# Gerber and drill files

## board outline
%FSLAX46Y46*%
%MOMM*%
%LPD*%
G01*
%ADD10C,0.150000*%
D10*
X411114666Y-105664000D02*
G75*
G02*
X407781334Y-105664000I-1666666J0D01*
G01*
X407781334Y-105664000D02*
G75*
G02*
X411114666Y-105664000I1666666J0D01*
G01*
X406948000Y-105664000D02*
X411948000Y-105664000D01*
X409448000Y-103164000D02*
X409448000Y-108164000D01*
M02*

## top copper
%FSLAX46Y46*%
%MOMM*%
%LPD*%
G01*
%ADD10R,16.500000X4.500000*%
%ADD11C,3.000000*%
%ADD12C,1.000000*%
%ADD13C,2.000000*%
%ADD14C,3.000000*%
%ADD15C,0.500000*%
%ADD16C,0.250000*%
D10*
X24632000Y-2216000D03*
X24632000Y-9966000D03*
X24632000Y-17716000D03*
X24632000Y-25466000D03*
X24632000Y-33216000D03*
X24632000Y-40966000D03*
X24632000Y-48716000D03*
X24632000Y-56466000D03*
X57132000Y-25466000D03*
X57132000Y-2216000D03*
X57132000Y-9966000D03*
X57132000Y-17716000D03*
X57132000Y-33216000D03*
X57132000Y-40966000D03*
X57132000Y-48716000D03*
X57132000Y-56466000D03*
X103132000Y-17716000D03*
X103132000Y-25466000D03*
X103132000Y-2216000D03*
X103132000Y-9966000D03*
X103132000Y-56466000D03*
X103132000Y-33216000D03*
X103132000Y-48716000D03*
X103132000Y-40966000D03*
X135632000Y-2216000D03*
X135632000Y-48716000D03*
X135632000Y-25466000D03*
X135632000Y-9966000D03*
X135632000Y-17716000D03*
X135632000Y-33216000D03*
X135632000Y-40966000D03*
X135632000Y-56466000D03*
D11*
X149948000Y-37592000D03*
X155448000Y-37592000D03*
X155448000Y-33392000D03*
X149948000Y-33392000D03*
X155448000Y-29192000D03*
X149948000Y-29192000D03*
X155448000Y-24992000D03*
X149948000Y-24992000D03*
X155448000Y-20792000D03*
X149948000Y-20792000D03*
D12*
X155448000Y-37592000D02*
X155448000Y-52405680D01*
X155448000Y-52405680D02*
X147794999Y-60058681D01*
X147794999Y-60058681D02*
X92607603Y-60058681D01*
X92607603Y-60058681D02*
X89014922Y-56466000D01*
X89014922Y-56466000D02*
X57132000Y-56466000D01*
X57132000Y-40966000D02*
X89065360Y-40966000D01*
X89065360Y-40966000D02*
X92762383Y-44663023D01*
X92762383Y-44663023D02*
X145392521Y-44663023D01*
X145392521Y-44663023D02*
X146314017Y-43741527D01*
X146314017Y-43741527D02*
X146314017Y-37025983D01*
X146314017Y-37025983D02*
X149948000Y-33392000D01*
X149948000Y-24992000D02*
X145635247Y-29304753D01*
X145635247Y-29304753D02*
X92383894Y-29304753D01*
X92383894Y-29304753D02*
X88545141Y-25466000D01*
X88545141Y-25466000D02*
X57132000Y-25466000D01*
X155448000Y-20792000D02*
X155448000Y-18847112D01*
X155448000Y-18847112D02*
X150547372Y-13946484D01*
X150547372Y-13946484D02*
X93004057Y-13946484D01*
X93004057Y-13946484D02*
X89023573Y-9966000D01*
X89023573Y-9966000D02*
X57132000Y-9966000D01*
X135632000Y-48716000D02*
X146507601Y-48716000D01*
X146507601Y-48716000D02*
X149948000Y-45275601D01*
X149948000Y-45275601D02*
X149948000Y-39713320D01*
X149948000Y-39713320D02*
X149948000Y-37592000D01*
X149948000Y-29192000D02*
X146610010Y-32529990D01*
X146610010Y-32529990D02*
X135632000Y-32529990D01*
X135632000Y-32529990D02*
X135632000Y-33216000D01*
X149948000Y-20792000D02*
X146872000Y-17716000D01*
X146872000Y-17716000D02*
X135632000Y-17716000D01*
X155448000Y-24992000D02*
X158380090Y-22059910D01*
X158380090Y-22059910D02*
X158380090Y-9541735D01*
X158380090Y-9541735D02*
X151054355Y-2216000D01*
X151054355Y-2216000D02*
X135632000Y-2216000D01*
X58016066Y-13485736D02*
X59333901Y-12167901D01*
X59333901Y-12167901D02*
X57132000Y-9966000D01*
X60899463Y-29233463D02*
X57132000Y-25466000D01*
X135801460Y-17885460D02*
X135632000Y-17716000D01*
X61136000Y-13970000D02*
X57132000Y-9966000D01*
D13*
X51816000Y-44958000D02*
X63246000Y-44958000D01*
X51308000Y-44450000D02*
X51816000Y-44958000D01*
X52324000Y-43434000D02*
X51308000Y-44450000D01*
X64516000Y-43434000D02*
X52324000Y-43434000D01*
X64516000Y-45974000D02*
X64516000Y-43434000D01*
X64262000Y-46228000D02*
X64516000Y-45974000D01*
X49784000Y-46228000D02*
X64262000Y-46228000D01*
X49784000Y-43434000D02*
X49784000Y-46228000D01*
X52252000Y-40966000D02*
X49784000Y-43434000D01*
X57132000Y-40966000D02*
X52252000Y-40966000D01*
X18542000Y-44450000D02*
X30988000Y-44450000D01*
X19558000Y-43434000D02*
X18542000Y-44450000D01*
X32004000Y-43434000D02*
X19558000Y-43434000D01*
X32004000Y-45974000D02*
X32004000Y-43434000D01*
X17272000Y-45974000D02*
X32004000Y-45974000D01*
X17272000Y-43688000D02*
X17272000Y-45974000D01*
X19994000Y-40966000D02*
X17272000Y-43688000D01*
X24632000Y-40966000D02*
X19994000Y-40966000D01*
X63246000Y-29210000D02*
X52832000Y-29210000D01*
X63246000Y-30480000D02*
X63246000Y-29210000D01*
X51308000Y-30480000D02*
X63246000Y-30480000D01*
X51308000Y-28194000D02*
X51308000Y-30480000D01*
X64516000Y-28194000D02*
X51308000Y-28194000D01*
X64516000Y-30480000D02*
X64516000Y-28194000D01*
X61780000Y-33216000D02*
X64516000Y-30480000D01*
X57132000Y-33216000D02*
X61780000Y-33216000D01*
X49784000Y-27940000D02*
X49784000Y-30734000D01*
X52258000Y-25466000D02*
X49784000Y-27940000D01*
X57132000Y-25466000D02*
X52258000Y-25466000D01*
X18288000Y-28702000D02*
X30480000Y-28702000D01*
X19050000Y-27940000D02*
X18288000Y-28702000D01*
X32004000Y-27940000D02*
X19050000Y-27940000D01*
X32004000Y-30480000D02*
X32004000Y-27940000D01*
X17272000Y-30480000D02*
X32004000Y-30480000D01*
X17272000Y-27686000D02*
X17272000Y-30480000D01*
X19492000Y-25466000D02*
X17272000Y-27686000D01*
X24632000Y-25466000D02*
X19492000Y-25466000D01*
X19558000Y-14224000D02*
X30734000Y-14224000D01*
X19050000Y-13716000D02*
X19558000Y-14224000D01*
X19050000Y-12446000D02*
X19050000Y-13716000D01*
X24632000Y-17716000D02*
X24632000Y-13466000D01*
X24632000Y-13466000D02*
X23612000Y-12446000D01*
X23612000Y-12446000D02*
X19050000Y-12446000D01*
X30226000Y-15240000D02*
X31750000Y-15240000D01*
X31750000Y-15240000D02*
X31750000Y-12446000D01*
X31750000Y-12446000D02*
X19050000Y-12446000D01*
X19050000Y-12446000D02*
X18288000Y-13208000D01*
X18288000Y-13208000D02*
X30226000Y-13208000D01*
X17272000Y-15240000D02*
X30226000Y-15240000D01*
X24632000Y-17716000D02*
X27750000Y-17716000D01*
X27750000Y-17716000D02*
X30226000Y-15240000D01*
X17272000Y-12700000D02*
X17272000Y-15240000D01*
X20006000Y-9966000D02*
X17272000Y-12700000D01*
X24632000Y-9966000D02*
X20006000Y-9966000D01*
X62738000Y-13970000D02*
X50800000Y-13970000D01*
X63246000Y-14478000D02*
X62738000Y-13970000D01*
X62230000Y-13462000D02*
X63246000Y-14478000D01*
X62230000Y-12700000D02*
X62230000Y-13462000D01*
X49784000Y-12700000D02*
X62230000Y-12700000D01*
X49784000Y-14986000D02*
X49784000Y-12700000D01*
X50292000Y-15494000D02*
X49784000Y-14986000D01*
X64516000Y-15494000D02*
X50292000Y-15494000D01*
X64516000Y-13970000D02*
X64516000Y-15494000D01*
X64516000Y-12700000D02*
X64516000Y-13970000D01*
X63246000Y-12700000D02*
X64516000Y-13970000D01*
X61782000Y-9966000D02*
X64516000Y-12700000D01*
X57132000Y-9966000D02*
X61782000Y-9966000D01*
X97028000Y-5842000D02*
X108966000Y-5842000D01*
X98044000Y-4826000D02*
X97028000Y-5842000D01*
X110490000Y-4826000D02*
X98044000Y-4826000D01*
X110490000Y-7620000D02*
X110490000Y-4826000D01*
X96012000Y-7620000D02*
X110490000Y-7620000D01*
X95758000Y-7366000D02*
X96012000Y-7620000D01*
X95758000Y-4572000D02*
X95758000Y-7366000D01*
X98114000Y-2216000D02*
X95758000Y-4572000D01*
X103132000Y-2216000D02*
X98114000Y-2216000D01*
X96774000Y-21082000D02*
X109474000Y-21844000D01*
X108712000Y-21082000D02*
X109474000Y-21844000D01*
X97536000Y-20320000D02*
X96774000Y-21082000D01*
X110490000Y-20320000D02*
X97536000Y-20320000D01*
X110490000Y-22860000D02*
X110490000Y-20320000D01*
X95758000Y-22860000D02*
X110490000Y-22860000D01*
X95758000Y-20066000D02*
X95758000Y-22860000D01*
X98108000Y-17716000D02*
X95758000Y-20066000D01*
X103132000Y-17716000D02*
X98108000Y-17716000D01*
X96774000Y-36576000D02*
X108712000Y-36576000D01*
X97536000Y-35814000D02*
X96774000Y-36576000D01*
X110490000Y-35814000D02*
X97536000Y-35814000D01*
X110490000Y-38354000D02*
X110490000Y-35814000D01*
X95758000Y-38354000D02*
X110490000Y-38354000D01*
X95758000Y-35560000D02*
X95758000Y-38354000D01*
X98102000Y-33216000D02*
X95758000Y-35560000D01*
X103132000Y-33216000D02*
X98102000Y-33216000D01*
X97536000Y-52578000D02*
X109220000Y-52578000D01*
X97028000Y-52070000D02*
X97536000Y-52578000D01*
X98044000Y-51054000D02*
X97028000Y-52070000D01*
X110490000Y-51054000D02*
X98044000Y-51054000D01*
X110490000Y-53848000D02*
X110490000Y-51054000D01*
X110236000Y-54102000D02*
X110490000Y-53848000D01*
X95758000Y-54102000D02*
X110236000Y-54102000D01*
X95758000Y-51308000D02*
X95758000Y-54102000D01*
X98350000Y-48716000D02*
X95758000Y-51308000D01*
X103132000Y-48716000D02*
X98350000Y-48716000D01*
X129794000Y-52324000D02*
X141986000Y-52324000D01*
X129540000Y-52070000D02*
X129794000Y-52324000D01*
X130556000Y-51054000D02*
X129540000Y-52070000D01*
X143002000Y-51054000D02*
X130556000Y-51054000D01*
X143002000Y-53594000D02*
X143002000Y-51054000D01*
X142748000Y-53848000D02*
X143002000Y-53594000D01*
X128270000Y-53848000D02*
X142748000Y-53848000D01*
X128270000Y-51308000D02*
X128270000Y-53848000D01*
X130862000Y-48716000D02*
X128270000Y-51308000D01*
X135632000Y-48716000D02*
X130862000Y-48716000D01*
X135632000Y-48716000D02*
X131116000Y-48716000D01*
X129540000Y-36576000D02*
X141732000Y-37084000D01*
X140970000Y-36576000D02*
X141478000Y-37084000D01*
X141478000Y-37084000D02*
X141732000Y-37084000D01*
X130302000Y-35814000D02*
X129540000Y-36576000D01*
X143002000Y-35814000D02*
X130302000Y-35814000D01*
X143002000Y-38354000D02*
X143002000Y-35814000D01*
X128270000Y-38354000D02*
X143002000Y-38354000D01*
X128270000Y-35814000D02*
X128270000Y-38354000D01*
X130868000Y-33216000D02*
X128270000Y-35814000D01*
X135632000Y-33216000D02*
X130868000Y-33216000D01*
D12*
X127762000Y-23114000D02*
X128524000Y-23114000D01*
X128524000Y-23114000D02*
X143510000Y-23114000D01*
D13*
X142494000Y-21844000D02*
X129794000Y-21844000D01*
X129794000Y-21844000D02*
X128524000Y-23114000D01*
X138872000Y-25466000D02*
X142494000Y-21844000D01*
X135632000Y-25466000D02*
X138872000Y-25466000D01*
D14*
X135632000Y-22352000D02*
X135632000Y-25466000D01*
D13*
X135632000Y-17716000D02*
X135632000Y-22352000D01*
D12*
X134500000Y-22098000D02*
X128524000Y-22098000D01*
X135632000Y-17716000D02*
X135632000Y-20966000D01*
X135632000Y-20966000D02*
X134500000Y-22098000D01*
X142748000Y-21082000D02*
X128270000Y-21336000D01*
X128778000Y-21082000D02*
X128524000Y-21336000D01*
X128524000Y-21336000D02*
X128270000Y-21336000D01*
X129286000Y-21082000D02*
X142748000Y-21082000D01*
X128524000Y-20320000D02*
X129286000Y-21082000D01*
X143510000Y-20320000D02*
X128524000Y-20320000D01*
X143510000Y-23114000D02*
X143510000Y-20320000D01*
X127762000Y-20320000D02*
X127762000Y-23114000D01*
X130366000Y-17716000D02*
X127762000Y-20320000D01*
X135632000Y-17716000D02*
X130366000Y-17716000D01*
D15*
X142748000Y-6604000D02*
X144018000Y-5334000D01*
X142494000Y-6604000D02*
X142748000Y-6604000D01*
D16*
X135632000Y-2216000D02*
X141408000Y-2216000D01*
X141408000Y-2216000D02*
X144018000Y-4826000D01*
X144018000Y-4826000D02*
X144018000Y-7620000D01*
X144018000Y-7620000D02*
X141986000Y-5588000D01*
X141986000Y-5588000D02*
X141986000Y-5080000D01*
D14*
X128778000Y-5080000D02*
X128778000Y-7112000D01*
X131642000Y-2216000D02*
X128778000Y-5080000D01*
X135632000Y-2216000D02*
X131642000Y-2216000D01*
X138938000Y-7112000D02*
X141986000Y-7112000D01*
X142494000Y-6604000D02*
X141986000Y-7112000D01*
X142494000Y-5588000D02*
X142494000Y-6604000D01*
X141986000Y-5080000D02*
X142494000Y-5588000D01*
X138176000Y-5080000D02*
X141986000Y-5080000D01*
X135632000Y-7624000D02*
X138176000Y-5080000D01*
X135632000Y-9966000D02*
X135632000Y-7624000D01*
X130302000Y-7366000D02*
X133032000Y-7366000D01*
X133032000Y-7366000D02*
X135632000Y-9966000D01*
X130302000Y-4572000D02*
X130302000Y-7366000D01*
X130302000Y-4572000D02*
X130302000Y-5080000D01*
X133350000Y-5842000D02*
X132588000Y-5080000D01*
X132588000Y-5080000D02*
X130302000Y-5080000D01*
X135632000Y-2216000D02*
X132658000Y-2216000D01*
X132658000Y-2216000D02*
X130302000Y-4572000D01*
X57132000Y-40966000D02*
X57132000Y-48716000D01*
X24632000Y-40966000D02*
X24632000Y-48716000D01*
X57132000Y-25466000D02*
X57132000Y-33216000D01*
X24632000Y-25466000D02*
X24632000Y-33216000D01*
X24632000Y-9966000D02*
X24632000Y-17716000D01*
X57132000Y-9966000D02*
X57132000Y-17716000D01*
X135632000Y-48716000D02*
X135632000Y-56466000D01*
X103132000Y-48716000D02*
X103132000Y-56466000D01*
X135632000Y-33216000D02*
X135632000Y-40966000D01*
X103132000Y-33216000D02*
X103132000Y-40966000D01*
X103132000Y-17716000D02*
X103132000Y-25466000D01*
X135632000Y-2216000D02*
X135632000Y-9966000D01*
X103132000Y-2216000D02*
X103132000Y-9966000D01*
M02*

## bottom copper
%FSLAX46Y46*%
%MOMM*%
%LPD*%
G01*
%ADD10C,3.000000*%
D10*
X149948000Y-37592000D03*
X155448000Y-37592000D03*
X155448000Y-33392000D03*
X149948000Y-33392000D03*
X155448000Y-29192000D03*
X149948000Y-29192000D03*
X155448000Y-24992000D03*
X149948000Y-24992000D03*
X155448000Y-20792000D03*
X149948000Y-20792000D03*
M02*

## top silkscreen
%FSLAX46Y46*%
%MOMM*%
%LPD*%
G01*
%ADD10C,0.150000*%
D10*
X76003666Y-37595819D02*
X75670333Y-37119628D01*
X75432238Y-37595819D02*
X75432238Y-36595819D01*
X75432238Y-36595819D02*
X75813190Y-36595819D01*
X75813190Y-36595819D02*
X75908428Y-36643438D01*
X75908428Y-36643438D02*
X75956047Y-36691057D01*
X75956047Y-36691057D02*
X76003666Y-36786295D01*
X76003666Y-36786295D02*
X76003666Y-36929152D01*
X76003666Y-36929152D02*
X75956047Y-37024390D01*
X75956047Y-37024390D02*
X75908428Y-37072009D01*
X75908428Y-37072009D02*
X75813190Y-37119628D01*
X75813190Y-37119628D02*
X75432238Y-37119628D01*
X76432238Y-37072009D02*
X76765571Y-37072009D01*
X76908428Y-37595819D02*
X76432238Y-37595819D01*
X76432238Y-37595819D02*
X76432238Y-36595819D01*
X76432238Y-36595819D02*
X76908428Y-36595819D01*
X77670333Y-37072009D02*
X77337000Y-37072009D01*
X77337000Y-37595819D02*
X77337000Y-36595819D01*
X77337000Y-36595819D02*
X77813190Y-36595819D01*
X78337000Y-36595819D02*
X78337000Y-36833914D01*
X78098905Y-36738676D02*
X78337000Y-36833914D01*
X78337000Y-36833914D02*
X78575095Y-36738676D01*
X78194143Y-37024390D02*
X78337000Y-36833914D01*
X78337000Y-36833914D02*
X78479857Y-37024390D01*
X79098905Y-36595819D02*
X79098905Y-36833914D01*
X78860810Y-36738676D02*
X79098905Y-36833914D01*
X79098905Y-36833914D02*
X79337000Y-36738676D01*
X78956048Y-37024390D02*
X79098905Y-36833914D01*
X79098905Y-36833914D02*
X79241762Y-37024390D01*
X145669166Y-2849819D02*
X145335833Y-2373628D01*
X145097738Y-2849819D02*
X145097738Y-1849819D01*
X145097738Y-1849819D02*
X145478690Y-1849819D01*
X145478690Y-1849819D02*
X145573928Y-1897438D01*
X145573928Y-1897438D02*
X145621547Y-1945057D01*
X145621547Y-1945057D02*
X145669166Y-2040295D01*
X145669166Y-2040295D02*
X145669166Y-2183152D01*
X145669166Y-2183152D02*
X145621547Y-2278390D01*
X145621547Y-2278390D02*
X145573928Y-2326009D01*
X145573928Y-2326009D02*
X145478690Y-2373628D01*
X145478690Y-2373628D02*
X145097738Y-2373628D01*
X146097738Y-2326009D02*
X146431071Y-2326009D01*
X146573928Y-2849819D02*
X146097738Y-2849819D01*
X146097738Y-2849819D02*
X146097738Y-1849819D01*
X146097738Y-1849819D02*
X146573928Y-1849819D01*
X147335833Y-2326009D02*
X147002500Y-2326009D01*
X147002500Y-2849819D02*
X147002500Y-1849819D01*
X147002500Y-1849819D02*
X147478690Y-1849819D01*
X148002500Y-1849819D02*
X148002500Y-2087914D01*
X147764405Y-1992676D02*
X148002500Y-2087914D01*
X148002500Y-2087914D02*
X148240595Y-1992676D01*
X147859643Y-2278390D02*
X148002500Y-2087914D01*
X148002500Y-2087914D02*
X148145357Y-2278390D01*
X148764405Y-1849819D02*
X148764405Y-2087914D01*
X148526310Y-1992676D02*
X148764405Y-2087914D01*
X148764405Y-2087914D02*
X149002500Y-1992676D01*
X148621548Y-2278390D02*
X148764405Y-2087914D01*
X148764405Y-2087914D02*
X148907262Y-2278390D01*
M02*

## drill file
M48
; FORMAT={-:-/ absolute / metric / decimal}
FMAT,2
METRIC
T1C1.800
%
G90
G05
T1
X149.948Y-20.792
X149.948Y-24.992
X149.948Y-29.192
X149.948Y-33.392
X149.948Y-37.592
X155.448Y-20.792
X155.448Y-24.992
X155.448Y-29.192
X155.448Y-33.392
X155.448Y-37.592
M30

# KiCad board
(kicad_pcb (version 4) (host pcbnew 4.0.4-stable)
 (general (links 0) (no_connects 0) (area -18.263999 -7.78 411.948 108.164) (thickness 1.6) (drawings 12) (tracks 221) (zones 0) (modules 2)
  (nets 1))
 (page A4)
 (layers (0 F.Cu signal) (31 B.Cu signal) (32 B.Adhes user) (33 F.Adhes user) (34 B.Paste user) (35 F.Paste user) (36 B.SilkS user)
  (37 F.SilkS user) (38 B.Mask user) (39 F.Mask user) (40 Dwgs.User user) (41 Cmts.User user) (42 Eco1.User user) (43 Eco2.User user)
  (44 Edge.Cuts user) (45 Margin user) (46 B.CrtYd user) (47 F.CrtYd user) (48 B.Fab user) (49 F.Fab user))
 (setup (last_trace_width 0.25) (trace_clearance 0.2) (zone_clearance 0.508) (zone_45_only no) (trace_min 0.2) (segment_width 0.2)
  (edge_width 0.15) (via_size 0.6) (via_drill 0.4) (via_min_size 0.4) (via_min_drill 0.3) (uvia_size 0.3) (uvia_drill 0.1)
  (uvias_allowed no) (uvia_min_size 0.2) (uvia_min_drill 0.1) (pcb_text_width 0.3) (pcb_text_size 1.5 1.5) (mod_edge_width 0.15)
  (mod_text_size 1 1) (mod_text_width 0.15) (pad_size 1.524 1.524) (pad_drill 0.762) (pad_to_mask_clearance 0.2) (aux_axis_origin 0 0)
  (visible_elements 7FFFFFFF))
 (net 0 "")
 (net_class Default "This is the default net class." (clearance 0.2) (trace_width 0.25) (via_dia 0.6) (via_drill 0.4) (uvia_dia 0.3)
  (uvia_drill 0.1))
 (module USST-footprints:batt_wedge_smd (layer F.Cu) (at 77.337 37.141)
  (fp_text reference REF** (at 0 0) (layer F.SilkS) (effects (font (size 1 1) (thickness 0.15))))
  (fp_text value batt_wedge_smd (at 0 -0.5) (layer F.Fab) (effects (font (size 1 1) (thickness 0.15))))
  (pad 1 smd rect (at -52.705 -34.925 90) (size 4.5 16.5) (layers F.Cu F.Paste F.Mask))
  (pad 2 smd rect (at -52.705 -27.175 90) (size 4.5 16.5) (layers F.Cu F.Paste F.Mask))
  (pad 3 smd rect (at -52.705 -19.425 90) (size 4.5 16.5) (layers F.Cu F.Paste F.Mask))
  (pad 4 smd rect (at -52.705 -11.675 90) (size 4.5 16.5) (layers F.Cu F.Paste F.Mask))
  (pad 5 smd rect (at -52.705 -3.925 90) (size 4.5 16.5) (layers F.Cu F.Paste F.Mask))
  (pad 6 smd rect (at -52.705 3.825 90) (size 4.5 16.5) (layers F.Cu F.Paste F.Mask))
  (pad 7 smd rect (at -52.705 11.575 90) (size 4.5 16.5) (layers F.Cu F.Paste F.Mask))
  (pad 8 smd rect (at -52.705 19.325 90) (size 4.5 16.5) (layers F.Cu F.Paste F.Mask))
  (pad 4 smd rect (at -20.205 -11.675 90) (size 4.5 16.5) (layers F.Cu F.Paste F.Mask))
  (pad 1 smd rect (at -20.205 -34.925 90) (size 4.5 16.5) (layers F.Cu F.Paste F.Mask))
  (pad 2 smd rect (at -20.205 -27.175 90) (size 4.5 16.5) (layers F.Cu F.Paste F.Mask))
  (pad 3 smd rect (at -20.205 -19.425 90) (size 4.5 16.5) (layers F.Cu F.Paste F.Mask))
  (pad 5 smd rect (at -20.205 -3.925 90) (size 4.5 16.5) (layers F.Cu F.Paste F.Mask))
  (pad 6 smd rect (at -20.205 3.825 90) (size 4.5 16.5) (layers F.Cu F.Paste F.Mask))
  (pad 7 smd rect (at -20.205 11.575 90) (size 4.5 16.5) (layers F.Cu F.Paste F.Mask))
  (pad 8 smd rect (at -20.205 19.325 90) (size 4.5 16.5) (layers F.Cu F.Paste F.Mask))
  (pad 3 smd rect (at 25.795 -19.425 90) (size 4.5 16.5) (layers F.Cu F.Paste F.Mask))
  (pad 4 smd rect (at 25.795 -11.675 90) (size 4.5 16.5) (layers F.Cu F.Paste F.Mask))
  (pad 1 smd rect (at 25.795 -34.925 90) (size 4.5 16.5) (layers F.Cu F.Paste F.Mask))
  (pad 2 smd rect (at 25.795 -27.175 90) (size 4.5 16.5) (layers F.Cu F.Paste F.Mask))
  (pad 8 smd rect (at 25.795 19.325 90) (size 4.5 16.5) (layers F.Cu F.Paste F.Mask))
  (pad 5 smd rect (at 25.795 -3.925 90) (size 4.5 16.5) (layers F.Cu F.Paste F.Mask))
  (pad 7 smd rect (at 25.795 11.575 90) (size 4.5 16.5) (layers F.Cu F.Paste F.Mask))
  (pad 6 smd rect (at 25.795 3.825 90) (size 4.5 16.5) (layers F.Cu F.Paste F.Mask))
  (pad 1 smd rect (at 58.295 -34.925 90) (size 4.5 16.5) (layers F.Cu F.Paste F.Mask))
  (pad 7 smd rect (at 58.295 11.575 90) (size 4.5 16.5) (layers F.Cu F.Paste F.Mask))
  (pad 4 smd rect (at 58.295 -11.675 90) (size 4.5 16.5) (layers F.Cu F.Paste F.Mask))
  (pad 2 smd rect (at 58.295 -27.175 90) (size 4.5 16.5) (layers F.Cu F.Paste F.Mask))
  (pad 3 smd rect (at 58.295 -19.425 90) (size 4.5 16.5) (layers F.Cu F.Paste F.Mask))
  (pad 5 smd rect (at 58.295 -3.925 90) (size 4.5 16.5) (layers F.Cu F.Paste F.Mask))
  (pad 6 smd rect (at 58.295 3.825 90) (size 4.5 16.5) (layers F.Cu F.Paste F.Mask))
  (pad 8 smd rect (at 58.295 19.325 90) (size 4.5 16.5) (layers F.Cu F.Paste F.Mask)))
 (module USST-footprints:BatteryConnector (layer F.Cu) (at 149.948 37.592)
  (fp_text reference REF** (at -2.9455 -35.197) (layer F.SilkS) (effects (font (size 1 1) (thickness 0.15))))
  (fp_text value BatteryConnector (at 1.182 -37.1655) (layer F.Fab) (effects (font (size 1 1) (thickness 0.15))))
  (pad "" np_thru_hole circle (at 0 0) (size 3 3) (drill 1.8) (layers *.Cu))
  (pad "" np_thru_hole circle (at 5.5 0) (size 3 3) (drill 1.8) (layers *.Cu))
  (pad "" np_thru_hole circle (at 5.5 -4.2) (size 3 3) (drill 1.8) (layers *.Cu))
  (pad "" np_thru_hole circle (at 0 -4.2) (size 3 3) (drill 1.8) (layers *.Cu))
  (pad "" np_thru_hole circle (at 5.5 -8.4) (size 3 3) (drill 1.8) (layers *.Cu))
  (pad "" np_thru_hole circle (at 0 -8.4) (size 3 3) (drill 1.8) (layers *.Cu))
  (pad "" np_thru_hole circle (at 5.5 -12.6) (size 3 3) (drill 1.8) (layers *.Cu))
  (pad "" np_thru_hole circle (at 0 -12.6) (size 3 3) (drill 1.8) (layers *.Cu))
  (pad "" np_thru_hole circle (at 5.5 -16.8) (size 3 3) (drill 1.8) (layers *.Cu))
  (pad "" np_thru_hole circle (at 0 -16.8) (size 3 3) (drill 1.8) (layers *.Cu)))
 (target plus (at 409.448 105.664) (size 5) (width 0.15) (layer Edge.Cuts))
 (segment (start 155.448 37.592) (end 155.448 52.40568) (width 1) (layer F.Cu) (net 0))
 (segment (start 155.448 52.40568) (end 147.794999 60.058681) (width 1) (layer F.Cu) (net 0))
 (segment (start 147.794999 60.058681) (end 92.607603 60.058681) (width 1) (layer F.Cu) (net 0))
 (segment (start 92.607603 60.058681) (end 89.014922 56.466) (width 1) (layer F.Cu) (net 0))
 (segment (start 89.014922 56.466) (end 57.132 56.466) (width 1) (layer F.Cu) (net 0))
 (segment (start 57.132 40.966) (end 89.06536 40.966) (width 1) (layer F.Cu) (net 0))
 (segment (start 89.06536 40.966) (end 92.762383 44.663023) (width 1) (layer F.Cu) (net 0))
 (segment (start 92.762383 44.663023) (end 145.392521 44.663023) (width 1) (layer F.Cu) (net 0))
 (segment (start 145.392521 44.663023) (end 146.314017 43.741527) (width 1) (layer F.Cu) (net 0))
 (segment (start 146.314017 43.741527) (end 146.314017 37.025983) (width 1) (layer F.Cu) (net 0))
 (segment (start 146.314017 37.025983) (end 149.948 33.392) (width 1) (layer F.Cu) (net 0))
 (segment (start 149.948 24.992) (end 145.635247 29.304753) (width 1) (layer F.Cu) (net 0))
 (segment (start 145.635247 29.304753) (end 92.383894 29.304753) (width 1) (layer F.Cu) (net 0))
 (segment (start 92.383894 29.304753) (end 88.545141 25.466) (width 1) (layer F.Cu) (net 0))
 (segment (start 88.545141 25.466) (end 57.132 25.466) (width 1) (layer F.Cu) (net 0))
 (segment (start 155.448 20.792) (end 155.448 18.847112) (width 1) (layer F.Cu) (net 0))
 (segment (start 155.448 18.847112) (end 150.547372 13.946484) (width 1) (layer F.Cu) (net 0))
 (segment (start 150.547372 13.946484) (end 93.004057 13.946484) (width 1) (layer F.Cu) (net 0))
 (segment (start 93.004057 13.946484) (end 89.023573 9.966) (width 1) (layer F.Cu) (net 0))
 (segment (start 89.023573 9.966) (end 57.132 9.966) (width 1) (layer F.Cu) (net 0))
 (segment (start 135.632 48.716) (end 146.507601 48.716) (width 1) (layer F.Cu) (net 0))
 (segment (start 146.507601 48.716) (end 149.948 45.275601) (width 1) (layer F.Cu) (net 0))
 (segment (start 149.948 45.275601) (end 149.948 39.71332) (width 1) (layer F.Cu) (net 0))
 (segment (start 149.948 39.71332) (end 149.948 37.592) (width 1) (layer F.Cu) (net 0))
 (segment (start 149.948 29.192) (end 146.61001 32.52999) (width 1) (layer F.Cu) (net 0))
 (segment (start 146.61001 32.52999) (end 135.632 32.52999) (width 1) (layer F.Cu) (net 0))
 (segment (start 135.632 32.52999) (end 135.632 33.216) (width 1) (layer F.Cu) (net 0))
 (segment (start 149.948 20.792) (end 146.872 17.716) (width 1) (layer F.Cu) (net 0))
 (segment (start 146.872 17.716) (end 135.632 17.716) (width 1) (layer F.Cu) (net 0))
 (segment (start 155.448 24.992) (end 158.38009 22.05991) (width 1) (layer F.Cu) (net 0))
 (segment (start 158.38009 22.05991) (end 158.38009 9.541735) (width 1) (layer F.Cu) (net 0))
 (segment (start 158.38009 9.541735) (end 151.054355 2.216) (width 1) (layer F.Cu) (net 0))
 (segment (start 151.054355 2.216) (end 135.632 2.216) (width 1) (layer F.Cu) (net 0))
 (segment (start 58.016066 13.485736) (end 59.333901 12.167901) (width 1) (layer F.Cu) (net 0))
 (segment (start 59.333901 12.167901) (end 57.132 9.966) (width 1) (layer F.Cu) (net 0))
 (segment (start 60.899463 29.233463) (end 57.132 25.466) (width 1) (layer F.Cu) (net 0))
 (segment (start 135.80146 17.88546) (end 135.632 17.716) (width 1) (layer F.Cu) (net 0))
 (segment (start 61.136 13.97) (end 57.132 9.966) (width 1) (layer F.Cu) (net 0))
 (segment (start 51.816 44.958) (end 63.246 44.958) (width 2) (layer F.Cu) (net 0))
 (segment (start 51.308 44.45) (end 51.816 44.958) (width 2) (layer F.Cu) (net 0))
 (segment (start 52.324 43.434) (end 51.308 44.45) (width 2) (layer F.Cu) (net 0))
 (segment (start 64.516 43.434) (end 52.324 43.434) (width 2) (layer F.Cu) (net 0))
 (segment (start 64.516 45.974) (end 64.516 43.434) (width 2) (layer F.Cu) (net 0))
 (segment (start 64.262 46.228) (end 64.516 45.974) (width 2) (layer F.Cu) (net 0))
 (segment (start 49.784 46.228) (end 64.262 46.228) (width 2) (layer F.Cu) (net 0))
 (segment (start 49.784 43.434) (end 49.784 46.228) (width 2) (layer F.Cu) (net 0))
 (segment (start 52.252 40.966) (end 49.784 43.434) (width 2) (layer F.Cu) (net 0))
 (segment (start 57.132 40.966) (end 52.252 40.966) (width 2) (layer F.Cu) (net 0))
 (segment (start 18.542 44.45) (end 30.988 44.45) (width 2) (layer F.Cu) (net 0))
 (segment (start 19.558 43.434) (end 18.542 44.45) (width 2) (layer F.Cu) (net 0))
 (segment (start 32.004 43.434) (end 19.558 43.434) (width 2) (layer F.Cu) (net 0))
 (segment (start 32.004 45.974) (end 32.004 43.434) (width 2) (layer F.Cu) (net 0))
 (segment (start 17.272 45.974) (end 32.004 45.974) (width 2) (layer F.Cu) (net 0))
 (segment (start 17.272 43.688) (end 17.272 45.974) (width 2) (layer F.Cu) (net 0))
 (segment (start 19.994 40.966) (end 17.272 43.688) (width 2) (layer F.Cu) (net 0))
 (segment (start 24.632 40.966) (end 19.994 40.966) (width 2) (layer F.Cu) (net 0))
 (segment (start 63.246 29.21) (end 52.832 29.21) (width 2) (layer F.Cu) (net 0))
 (segment (start 63.246 30.48) (end 63.246 29.21) (width 2) (layer F.Cu) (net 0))
 (segment (start 51.308 30.48) (end 63.246 30.48) (width 2) (layer F.Cu) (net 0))
 (segment (start 51.308 28.194) (end 51.308 30.48) (width 2) (layer F.Cu) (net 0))
 (segment (start 64.516 28.194) (end 51.308 28.194) (width 2) (layer F.Cu) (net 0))
 (segment (start 64.516 30.48) (end 64.516 28.194) (width 2) (layer F.Cu) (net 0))
 (segment (start 61.78 33.216) (end 64.516 30.48) (width 2) (layer F.Cu) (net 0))
 (segment (start 57.132 33.216) (end 61.78 33.216) (width 2) (layer F.Cu) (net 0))
 (segment (start 49.784 27.94) (end 49.784 30.734) (width 2) (layer F.Cu) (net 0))
 (segment (start 52.258 25.466) (end 49.784 27.94) (width 2) (layer F.Cu) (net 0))
 (segment (start 57.132 25.466) (end 52.258 25.466) (width 2) (layer F.Cu) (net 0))
 (segment (start 18.288 28.702) (end 30.48 28.702) (width 2) (layer F.Cu) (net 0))
 (segment (start 19.05 27.94) (end 18.288 28.702) (width 2) (layer F.Cu) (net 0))
 (segment (start 32.004 27.94) (end 19.05 27.94) (width 2) (layer F.Cu) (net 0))
 (segment (start 32.004 30.48) (end 32.004 27.94) (width 2) (layer F.Cu) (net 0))
 (segment (start 17.272 30.48) (end 32.004 30.48) (width 2) (layer F.Cu) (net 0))
 (segment (start 17.272 27.686) (end 17.272 30.48) (width 2) (layer F.Cu) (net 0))
 (segment (start 19.492 25.466) (end 17.272 27.686) (width 2) (layer F.Cu) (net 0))
 (segment (start 24.632 25.466) (end 19.492 25.466) (width 2) (layer F.Cu) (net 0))
 (segment (start 19.558 14.224) (end 30.734 14.224) (width 2) (layer F.Cu) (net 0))
 (segment (start 19.05 13.716) (end 19.558 14.224) (width 2) (layer F.Cu) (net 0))
 (segment (start 19.05 12.446) (end 19.05 13.716) (width 2) (layer F.Cu) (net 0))
 (segment (start 24.632 17.716) (end 24.632 13.466) (width 2) (layer F.Cu) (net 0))
 (segment (start 24.632 13.466) (end 23.612 12.446) (width 2) (layer F.Cu) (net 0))
 (segment (start 23.612 12.446) (end 19.05 12.446) (width 2) (layer F.Cu) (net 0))
 (segment (start 30.226 15.24) (end 31.75 15.24) (width 2) (layer F.Cu) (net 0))
 (segment (start 31.75 15.24) (end 31.75 12.446) (width 2) (layer F.Cu) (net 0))
 (segment (start 31.75 12.446) (end 19.05 12.446) (width 2) (layer F.Cu) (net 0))
 (segment (start 19.05 12.446) (end 18.288 13.208) (width 2) (layer F.Cu) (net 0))
 (segment (start 18.288 13.208) (end 30.226 13.208) (width 2) (layer F.Cu) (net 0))
 (segment (start 17.272 15.24) (end 30.226 15.24) (width 2) (layer F.Cu) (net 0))
 (segment (start 24.632 17.716) (end 27.75 17.716) (width 2) (layer F.Cu) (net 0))
 (segment (start 27.75 17.716) (end 30.226 15.24) (width 2) (layer F.Cu) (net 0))
 (segment (start 17.272 12.7) (end 17.272 15.24) (width 2) (layer F.Cu) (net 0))
 (segment (start 20.006 9.966) (end 17.272 12.7) (width 2) (layer F.Cu) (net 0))
 (segment (start 24.632 9.966) (end 20.006 9.966) (width 2) (layer F.Cu) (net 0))
 (segment (start 62.738 13.97) (end 50.8 13.97) (width 2) (layer F.Cu) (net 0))
 (segment (start 63.246 14.478) (end 62.738 13.97) (width 2) (layer F.Cu) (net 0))
 (segment (start 62.23 13.462) (end 63.246 14.478) (width 2) (layer F.Cu) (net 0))
 (segment (start 62.23 12.7) (end 62.23 13.462) (width 2) (layer F.Cu) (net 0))
 (segment (start 49.784 12.7) (end 62.23 12.7) (width 2) (layer F.Cu) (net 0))
 (segment (start 49.784 14.986) (end 49.784 12.7) (width 2) (layer F.Cu) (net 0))
 (segment (start 50.292 15.494) (end 49.784 14.986) (width 2) (layer F.Cu) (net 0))
 (segment (start 64.516 15.494) (end 50.292 15.494) (width 2) (layer F.Cu) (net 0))
 (segment (start 64.516 13.97) (end 64.516 15.494) (width 2) (layer F.Cu) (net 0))
 (segment (start 64.516 12.7) (end 64.516 13.97) (width 2) (layer F.Cu) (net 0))
 (segment (start 63.246 12.7) (end 64.516 13.97) (width 2) (layer F.Cu) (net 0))
 (segment (start 61.782 9.966) (end 64.516 12.7) (width 2) (layer F.Cu) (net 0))
 (segment (start 57.132 9.966) (end 61.782 9.966) (width 2) (layer F.Cu) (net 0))
 (segment (start 97.028 5.842) (end 108.966 5.842) (width 2) (layer F.Cu) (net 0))
 (segment (start 98.044 4.826) (end 97.028 5.842) (width 2) (layer F.Cu) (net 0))
 (segment (start 110.49 4.826) (end 98.044 4.826) (width 2) (layer F.Cu) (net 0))
 (segment (start 110.49 7.62) (end 110.49 4.826) (width 2) (layer F.Cu) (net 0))
 (segment (start 96.012 7.62) (end 110.49 7.62) (width 2) (layer F.Cu) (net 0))
 (segment (start 95.758 7.366) (end 96.012 7.62) (width 2) (layer F.Cu) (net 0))
 (segment (start 95.758 4.572) (end 95.758 7.366) (width 2) (layer F.Cu) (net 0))
 (segment (start 98.114 2.216) (end 95.758 4.572) (width 2) (layer F.Cu) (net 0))
 (segment (start 103.132 2.216) (end 98.114 2.216) (width 2) (layer F.Cu) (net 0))
 (segment (start 96.774 21.082) (end 109.474 21.844) (width 2) (layer F.Cu) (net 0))
 (segment (start 108.712 21.082) (end 109.474 21.844) (width 2) (layer F.Cu) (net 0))
 (segment (start 97.536 20.32) (end 96.774 21.082) (width 2) (layer F.Cu) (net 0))
 (segment (start 110.49 20.32) (end 97.536 20.32) (width 2) (layer F.Cu) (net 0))
 (segment (start 110.49 22.86) (end 110.49 20.32) (width 2) (layer F.Cu) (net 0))
 (segment (start 95.758 22.86) (end 110.49 22.86) (width 2) (layer F.Cu) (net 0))
 (segment (start 95.758 20.066) (end 95.758 22.86) (width 2) (layer F.Cu) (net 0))
 (segment (start 98.108 17.716) (end 95.758 20.066) (width 2) (layer F.Cu) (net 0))
 (segment (start 103.132 17.716) (end 98.108 17.716) (width 2) (layer F.Cu) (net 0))
 (segment (start 96.774 36.576) (end 108.712 36.576) (width 2) (layer F.Cu) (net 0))
 (segment (start 97.536 35.814) (end 96.774 36.576) (width 2) (layer F.Cu) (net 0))
 (segment (start 110.49 35.814) (end 97.536 35.814) (width 2) (layer F.Cu) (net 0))
 (segment (start 110.49 38.354) (end 110.49 35.814) (width 2) (layer F.Cu) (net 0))
 (segment (start 95.758 38.354) (end 110.49 38.354) (width 2) (layer F.Cu) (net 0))
 (segment (start 95.758 35.56) (end 95.758 38.354) (width 2) (layer F.Cu) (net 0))
 (segment (start 98.102 33.216) (end 95.758 35.56) (width 2) (layer F.Cu) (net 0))
 (segment (start 103.132 33.216) (end 98.102 33.216) (width 2) (layer F.Cu) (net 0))
 (segment (start 97.536 52.578) (end 109.22 52.578) (width 2) (layer F.Cu) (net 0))
 (segment (start 97.028 52.07) (end 97.536 52.578) (width 2) (layer F.Cu) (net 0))
 (segment (start 98.044 51.054) (end 97.028 52.07) (width 2) (layer F.Cu) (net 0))
 (segment (start 110.49 51.054) (end 98.044 51.054) (width 2) (layer F.Cu) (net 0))
 (segment (start 110.49 53.848) (end 110.49 51.054) (width 2) (layer F.Cu) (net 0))
 (segment (start 110.236 54.102) (end 110.49 53.848) (width 2) (layer F.Cu) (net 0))
 (segment (start 95.758 54.102) (end 110.236 54.102) (width 2) (layer F.Cu) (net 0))
 (segment (start 95.758 51.308) (end 95.758 54.102) (width 2) (layer F.Cu) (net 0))
 (segment (start 98.35 48.716) (end 95.758 51.308) (width 2) (layer F.Cu) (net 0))
 (segment (start 103.132 48.716) (end 98.35 48.716) (width 2) (layer F.Cu) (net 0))
 (segment (start 129.794 52.324) (end 141.986 52.324) (width 2) (layer F.Cu) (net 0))
 (segment (start 129.54 52.07) (end 129.794 52.324) (width 2) (layer F.Cu) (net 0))
 (segment (start 130.556 51.054) (end 129.54 52.07) (width 2) (layer F.Cu) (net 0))
 (segment (start 143.002 51.054) (end 130.556 51.054) (width 2) (layer F.Cu) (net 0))
 (segment (start 143.002 53.594) (end 143.002 51.054) (width 2) (layer F.Cu) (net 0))
 (segment (start 142.748 53.848) (end 143.002 53.594) (width 2) (layer F.Cu) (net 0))
 (segment (start 128.27 53.848) (end 142.748 53.848) (width 2) (layer F.Cu) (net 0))
 (segment (start 128.27 51.308) (end 128.27 53.848) (width 2) (layer F.Cu) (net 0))
 (segment (start 130.862 48.716) (end 128.27 51.308) (width 2) (layer F.Cu) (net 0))
 (segment (start 135.632 48.716) (end 130.862 48.716) (width 2) (layer F.Cu) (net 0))
 (segment (start 135.632 48.716) (end 131.116 48.716) (width 2) (layer F.Cu) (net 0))
 (segment (start 129.54 36.576) (end 141.732 37.084) (width 2) (layer F.Cu) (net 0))
 (segment (start 140.97 36.576) (end 141.478 37.084) (width 2) (layer F.Cu) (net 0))
 (segment (start 141.478 37.084) (end 141.732 37.084) (width 2) (layer F.Cu) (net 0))
 (segment (start 130.302 35.814) (end 129.54 36.576) (width 2) (layer F.Cu) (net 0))
 (segment (start 143.002 35.814) (end 130.302 35.814) (width 2) (layer F.Cu) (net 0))
 (segment (start 143.002 38.354) (end 143.002 35.814) (width 2) (layer F.Cu) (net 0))
 (segment (start 128.27 38.354) (end 143.002 38.354) (width 2) (layer F.Cu) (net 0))
 (segment (start 128.27 35.814) (end 128.27 38.354) (width 2) (layer F.Cu) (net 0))
 (segment (start 130.868 33.216) (end 128.27 35.814) (width 2) (layer F.Cu) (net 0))
 (segment (start 135.632 33.216) (end 130.868 33.216) (width 2) (layer F.Cu) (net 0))
 (segment (start 127.762 23.114) (end 128.524 23.114) (width 1) (layer F.Cu) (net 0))
 (segment (start 128.524 23.114) (end 143.51 23.114) (width 1) (layer F.Cu) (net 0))
 (segment (start 142.494 21.844) (end 129.794 21.844) (width 2) (layer F.Cu) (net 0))
 (segment (start 129.794 21.844) (end 128.524 23.114) (width 2) (layer F.Cu) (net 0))
 (segment (start 138.872 25.466) (end 142.494 21.844) (width 2) (layer F.Cu) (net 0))
 (segment (start 135.632 25.466) (end 138.872 25.466) (width 2) (layer F.Cu) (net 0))
 (segment (start 135.632 22.352) (end 135.632 25.466) (width 3) (layer F.Cu) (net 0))
 (segment (start 135.632 17.716) (end 135.632 22.352) (width 2) (layer F.Cu) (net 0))
 (segment (start 134.5 22.098) (end 128.524 22.098) (width 1) (layer F.Cu) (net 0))
 (segment (start 135.632 17.716) (end 135.632 20.966) (width 1) (layer F.Cu) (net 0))
 (segment (start 135.632 20.966) (end 134.5 22.098) (width 1) (layer F.Cu) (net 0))
 (segment (start 142.748 21.082) (end 128.27 21.336) (width 1) (layer F.Cu) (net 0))
 (segment (start 128.778 21.082) (end 128.524 21.336) (width 1) (layer F.Cu) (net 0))
 (segment (start 128.524 21.336) (end 128.27 21.336) (width 1) (layer F.Cu) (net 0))
 (segment (start 129.286 21.082) (end 142.748 21.082) (width 1) (layer F.Cu) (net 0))
 (segment (start 128.524 20.32) (end 129.286 21.082) (width 1) (layer F.Cu) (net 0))
 (segment (start 143.51 20.32) (end 128.524 20.32) (width 1) (layer F.Cu) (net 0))
 (segment (start 143.51 23.114) (end 143.51 20.32) (width 1) (layer F.Cu) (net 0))
 (segment (start 127.762 20.32) (end 127.762 23.114) (width 1) (layer F.Cu) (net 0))
 (segment (start 130.366 17.716) (end 127.762 20.32) (width 1) (layer F.Cu) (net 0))
 (segment (start 135.632 17.716) (end 130.366 17.716) (width 1) (layer F.Cu) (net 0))
 (segment (start 142.748 6.604) (end 144.018 5.334) (width 0.5) (layer F.Cu) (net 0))
 (segment (start 142.494 6.604) (end 142.748 6.604) (width 0.5) (layer F.Cu) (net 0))
 (segment (start 135.632 2.216) (end 141.408 2.216) (width 0.25) (layer F.Cu) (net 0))
 (segment (start 141.408 2.216) (end 144.018 4.826) (width 0.25) (layer F.Cu) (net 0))
 (segment (start 144.018 4.826) (end 144.018 7.62) (width 0.25) (layer F.Cu) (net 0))
 (segment (start 144.018 7.62) (end 141.986 5.588) (width 0.25) (layer F.Cu) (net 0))
 (segment (start 141.986 5.588) (end 141.986 5.08) (width 0.25) (layer F.Cu) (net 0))
 (segment (start 128.778 5.08) (end 128.778 7.112) (width 3) (layer F.Cu) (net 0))
 (segment (start 131.642 2.216) (end 128.778 5.08) (width 3) (layer F.Cu) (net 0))
 (segment (start 135.632 2.216) (end 131.642 2.216) (width 3) (layer F.Cu) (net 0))
 (segment (start 138.938 7.112) (end 141.986 7.112) (width 3) (layer F.Cu) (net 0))
 (segment (start 142.494 6.604) (end 141.986 7.112) (width 3) (layer F.Cu) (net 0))
 (segment (start 142.494 5.588) (end 142.494 6.604) (width 3) (layer F.Cu) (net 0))
 (segment (start 141.986 5.08) (end 142.494 5.588) (width 3) (layer F.Cu) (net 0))
 (segment (start 138.176 5.08) (end 141.986 5.08) (width 3) (layer F.Cu) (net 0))
 (segment (start 135.632 7.624) (end 138.176 5.08) (width 3) (layer F.Cu) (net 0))
 (segment (start 135.632 9.966) (end 135.632 7.624) (width 3) (layer F.Cu) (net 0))
 (segment (start 130.302 7.366) (end 133.032 7.366) (width 3) (layer F.Cu) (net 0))
 (segment (start 133.032 7.366) (end 135.632 9.966) (width 3) (layer F.Cu) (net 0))
 (segment (start 130.302 4.572) (end 130.302 7.366) (width 3) (layer F.Cu) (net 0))
 (segment (start 130.302 4.572) (end 130.302 5.08) (width 3) (layer F.Cu) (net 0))
 (segment (start 133.35 5.842) (end 132.588 5.08) (width 3) (layer F.Cu) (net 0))
 (segment (start 132.588 5.08) (end 130.302 5.08) (width 3) (layer F.Cu) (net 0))
 (segment (start 135.632 2.216) (end 132.658 2.216) (width 3) (layer F.Cu) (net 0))
 (segment (start 132.658 2.216) (end 130.302 4.572) (width 3) (layer F.Cu) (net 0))
 (segment (start 57.132 40.966) (end 57.132 48.716) (width 3) (layer F.Cu) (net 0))
 (segment (start 24.632 40.966) (end 24.632 48.716) (width 3) (layer F.Cu) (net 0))
 (segment (start 57.132 25.466) (end 57.132 33.216) (width 3) (layer F.Cu) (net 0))
 (segment (start 24.632 25.466) (end 24.632 33.216) (width 3) (layer F.Cu) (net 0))
 (segment (start 24.632 9.966) (end 24.632 17.716) (width 3) (layer F.Cu) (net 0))
 (segment (start 57.132 9.966) (end 57.132 17.716) (width 3) (layer F.Cu) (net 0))
 (segment (start 135.632 48.716) (end 135.632 56.466) (width 3) (layer F.Cu) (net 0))
 (segment (start 103.132 48.716) (end 103.132 56.466) (width 3) (layer F.Cu) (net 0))
 (segment (start 135.632 33.216) (end 135.632 40.966) (width 3) (layer F.Cu) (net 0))
 (segment (start 103.132 33.216) (end 103.132 40.966) (width 3) (layer F.Cu) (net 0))
 (segment (start 103.132 17.716) (end 103.132 25.466) (width 3) (layer F.Cu) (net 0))
 (segment (start 135.632 2.216) (end 135.632 9.966) (width 3) (layer F.Cu) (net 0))
 (segment (start 103.132 2.216) (end 103.132 9.966) (width 3) (layer F.Cu) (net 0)))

